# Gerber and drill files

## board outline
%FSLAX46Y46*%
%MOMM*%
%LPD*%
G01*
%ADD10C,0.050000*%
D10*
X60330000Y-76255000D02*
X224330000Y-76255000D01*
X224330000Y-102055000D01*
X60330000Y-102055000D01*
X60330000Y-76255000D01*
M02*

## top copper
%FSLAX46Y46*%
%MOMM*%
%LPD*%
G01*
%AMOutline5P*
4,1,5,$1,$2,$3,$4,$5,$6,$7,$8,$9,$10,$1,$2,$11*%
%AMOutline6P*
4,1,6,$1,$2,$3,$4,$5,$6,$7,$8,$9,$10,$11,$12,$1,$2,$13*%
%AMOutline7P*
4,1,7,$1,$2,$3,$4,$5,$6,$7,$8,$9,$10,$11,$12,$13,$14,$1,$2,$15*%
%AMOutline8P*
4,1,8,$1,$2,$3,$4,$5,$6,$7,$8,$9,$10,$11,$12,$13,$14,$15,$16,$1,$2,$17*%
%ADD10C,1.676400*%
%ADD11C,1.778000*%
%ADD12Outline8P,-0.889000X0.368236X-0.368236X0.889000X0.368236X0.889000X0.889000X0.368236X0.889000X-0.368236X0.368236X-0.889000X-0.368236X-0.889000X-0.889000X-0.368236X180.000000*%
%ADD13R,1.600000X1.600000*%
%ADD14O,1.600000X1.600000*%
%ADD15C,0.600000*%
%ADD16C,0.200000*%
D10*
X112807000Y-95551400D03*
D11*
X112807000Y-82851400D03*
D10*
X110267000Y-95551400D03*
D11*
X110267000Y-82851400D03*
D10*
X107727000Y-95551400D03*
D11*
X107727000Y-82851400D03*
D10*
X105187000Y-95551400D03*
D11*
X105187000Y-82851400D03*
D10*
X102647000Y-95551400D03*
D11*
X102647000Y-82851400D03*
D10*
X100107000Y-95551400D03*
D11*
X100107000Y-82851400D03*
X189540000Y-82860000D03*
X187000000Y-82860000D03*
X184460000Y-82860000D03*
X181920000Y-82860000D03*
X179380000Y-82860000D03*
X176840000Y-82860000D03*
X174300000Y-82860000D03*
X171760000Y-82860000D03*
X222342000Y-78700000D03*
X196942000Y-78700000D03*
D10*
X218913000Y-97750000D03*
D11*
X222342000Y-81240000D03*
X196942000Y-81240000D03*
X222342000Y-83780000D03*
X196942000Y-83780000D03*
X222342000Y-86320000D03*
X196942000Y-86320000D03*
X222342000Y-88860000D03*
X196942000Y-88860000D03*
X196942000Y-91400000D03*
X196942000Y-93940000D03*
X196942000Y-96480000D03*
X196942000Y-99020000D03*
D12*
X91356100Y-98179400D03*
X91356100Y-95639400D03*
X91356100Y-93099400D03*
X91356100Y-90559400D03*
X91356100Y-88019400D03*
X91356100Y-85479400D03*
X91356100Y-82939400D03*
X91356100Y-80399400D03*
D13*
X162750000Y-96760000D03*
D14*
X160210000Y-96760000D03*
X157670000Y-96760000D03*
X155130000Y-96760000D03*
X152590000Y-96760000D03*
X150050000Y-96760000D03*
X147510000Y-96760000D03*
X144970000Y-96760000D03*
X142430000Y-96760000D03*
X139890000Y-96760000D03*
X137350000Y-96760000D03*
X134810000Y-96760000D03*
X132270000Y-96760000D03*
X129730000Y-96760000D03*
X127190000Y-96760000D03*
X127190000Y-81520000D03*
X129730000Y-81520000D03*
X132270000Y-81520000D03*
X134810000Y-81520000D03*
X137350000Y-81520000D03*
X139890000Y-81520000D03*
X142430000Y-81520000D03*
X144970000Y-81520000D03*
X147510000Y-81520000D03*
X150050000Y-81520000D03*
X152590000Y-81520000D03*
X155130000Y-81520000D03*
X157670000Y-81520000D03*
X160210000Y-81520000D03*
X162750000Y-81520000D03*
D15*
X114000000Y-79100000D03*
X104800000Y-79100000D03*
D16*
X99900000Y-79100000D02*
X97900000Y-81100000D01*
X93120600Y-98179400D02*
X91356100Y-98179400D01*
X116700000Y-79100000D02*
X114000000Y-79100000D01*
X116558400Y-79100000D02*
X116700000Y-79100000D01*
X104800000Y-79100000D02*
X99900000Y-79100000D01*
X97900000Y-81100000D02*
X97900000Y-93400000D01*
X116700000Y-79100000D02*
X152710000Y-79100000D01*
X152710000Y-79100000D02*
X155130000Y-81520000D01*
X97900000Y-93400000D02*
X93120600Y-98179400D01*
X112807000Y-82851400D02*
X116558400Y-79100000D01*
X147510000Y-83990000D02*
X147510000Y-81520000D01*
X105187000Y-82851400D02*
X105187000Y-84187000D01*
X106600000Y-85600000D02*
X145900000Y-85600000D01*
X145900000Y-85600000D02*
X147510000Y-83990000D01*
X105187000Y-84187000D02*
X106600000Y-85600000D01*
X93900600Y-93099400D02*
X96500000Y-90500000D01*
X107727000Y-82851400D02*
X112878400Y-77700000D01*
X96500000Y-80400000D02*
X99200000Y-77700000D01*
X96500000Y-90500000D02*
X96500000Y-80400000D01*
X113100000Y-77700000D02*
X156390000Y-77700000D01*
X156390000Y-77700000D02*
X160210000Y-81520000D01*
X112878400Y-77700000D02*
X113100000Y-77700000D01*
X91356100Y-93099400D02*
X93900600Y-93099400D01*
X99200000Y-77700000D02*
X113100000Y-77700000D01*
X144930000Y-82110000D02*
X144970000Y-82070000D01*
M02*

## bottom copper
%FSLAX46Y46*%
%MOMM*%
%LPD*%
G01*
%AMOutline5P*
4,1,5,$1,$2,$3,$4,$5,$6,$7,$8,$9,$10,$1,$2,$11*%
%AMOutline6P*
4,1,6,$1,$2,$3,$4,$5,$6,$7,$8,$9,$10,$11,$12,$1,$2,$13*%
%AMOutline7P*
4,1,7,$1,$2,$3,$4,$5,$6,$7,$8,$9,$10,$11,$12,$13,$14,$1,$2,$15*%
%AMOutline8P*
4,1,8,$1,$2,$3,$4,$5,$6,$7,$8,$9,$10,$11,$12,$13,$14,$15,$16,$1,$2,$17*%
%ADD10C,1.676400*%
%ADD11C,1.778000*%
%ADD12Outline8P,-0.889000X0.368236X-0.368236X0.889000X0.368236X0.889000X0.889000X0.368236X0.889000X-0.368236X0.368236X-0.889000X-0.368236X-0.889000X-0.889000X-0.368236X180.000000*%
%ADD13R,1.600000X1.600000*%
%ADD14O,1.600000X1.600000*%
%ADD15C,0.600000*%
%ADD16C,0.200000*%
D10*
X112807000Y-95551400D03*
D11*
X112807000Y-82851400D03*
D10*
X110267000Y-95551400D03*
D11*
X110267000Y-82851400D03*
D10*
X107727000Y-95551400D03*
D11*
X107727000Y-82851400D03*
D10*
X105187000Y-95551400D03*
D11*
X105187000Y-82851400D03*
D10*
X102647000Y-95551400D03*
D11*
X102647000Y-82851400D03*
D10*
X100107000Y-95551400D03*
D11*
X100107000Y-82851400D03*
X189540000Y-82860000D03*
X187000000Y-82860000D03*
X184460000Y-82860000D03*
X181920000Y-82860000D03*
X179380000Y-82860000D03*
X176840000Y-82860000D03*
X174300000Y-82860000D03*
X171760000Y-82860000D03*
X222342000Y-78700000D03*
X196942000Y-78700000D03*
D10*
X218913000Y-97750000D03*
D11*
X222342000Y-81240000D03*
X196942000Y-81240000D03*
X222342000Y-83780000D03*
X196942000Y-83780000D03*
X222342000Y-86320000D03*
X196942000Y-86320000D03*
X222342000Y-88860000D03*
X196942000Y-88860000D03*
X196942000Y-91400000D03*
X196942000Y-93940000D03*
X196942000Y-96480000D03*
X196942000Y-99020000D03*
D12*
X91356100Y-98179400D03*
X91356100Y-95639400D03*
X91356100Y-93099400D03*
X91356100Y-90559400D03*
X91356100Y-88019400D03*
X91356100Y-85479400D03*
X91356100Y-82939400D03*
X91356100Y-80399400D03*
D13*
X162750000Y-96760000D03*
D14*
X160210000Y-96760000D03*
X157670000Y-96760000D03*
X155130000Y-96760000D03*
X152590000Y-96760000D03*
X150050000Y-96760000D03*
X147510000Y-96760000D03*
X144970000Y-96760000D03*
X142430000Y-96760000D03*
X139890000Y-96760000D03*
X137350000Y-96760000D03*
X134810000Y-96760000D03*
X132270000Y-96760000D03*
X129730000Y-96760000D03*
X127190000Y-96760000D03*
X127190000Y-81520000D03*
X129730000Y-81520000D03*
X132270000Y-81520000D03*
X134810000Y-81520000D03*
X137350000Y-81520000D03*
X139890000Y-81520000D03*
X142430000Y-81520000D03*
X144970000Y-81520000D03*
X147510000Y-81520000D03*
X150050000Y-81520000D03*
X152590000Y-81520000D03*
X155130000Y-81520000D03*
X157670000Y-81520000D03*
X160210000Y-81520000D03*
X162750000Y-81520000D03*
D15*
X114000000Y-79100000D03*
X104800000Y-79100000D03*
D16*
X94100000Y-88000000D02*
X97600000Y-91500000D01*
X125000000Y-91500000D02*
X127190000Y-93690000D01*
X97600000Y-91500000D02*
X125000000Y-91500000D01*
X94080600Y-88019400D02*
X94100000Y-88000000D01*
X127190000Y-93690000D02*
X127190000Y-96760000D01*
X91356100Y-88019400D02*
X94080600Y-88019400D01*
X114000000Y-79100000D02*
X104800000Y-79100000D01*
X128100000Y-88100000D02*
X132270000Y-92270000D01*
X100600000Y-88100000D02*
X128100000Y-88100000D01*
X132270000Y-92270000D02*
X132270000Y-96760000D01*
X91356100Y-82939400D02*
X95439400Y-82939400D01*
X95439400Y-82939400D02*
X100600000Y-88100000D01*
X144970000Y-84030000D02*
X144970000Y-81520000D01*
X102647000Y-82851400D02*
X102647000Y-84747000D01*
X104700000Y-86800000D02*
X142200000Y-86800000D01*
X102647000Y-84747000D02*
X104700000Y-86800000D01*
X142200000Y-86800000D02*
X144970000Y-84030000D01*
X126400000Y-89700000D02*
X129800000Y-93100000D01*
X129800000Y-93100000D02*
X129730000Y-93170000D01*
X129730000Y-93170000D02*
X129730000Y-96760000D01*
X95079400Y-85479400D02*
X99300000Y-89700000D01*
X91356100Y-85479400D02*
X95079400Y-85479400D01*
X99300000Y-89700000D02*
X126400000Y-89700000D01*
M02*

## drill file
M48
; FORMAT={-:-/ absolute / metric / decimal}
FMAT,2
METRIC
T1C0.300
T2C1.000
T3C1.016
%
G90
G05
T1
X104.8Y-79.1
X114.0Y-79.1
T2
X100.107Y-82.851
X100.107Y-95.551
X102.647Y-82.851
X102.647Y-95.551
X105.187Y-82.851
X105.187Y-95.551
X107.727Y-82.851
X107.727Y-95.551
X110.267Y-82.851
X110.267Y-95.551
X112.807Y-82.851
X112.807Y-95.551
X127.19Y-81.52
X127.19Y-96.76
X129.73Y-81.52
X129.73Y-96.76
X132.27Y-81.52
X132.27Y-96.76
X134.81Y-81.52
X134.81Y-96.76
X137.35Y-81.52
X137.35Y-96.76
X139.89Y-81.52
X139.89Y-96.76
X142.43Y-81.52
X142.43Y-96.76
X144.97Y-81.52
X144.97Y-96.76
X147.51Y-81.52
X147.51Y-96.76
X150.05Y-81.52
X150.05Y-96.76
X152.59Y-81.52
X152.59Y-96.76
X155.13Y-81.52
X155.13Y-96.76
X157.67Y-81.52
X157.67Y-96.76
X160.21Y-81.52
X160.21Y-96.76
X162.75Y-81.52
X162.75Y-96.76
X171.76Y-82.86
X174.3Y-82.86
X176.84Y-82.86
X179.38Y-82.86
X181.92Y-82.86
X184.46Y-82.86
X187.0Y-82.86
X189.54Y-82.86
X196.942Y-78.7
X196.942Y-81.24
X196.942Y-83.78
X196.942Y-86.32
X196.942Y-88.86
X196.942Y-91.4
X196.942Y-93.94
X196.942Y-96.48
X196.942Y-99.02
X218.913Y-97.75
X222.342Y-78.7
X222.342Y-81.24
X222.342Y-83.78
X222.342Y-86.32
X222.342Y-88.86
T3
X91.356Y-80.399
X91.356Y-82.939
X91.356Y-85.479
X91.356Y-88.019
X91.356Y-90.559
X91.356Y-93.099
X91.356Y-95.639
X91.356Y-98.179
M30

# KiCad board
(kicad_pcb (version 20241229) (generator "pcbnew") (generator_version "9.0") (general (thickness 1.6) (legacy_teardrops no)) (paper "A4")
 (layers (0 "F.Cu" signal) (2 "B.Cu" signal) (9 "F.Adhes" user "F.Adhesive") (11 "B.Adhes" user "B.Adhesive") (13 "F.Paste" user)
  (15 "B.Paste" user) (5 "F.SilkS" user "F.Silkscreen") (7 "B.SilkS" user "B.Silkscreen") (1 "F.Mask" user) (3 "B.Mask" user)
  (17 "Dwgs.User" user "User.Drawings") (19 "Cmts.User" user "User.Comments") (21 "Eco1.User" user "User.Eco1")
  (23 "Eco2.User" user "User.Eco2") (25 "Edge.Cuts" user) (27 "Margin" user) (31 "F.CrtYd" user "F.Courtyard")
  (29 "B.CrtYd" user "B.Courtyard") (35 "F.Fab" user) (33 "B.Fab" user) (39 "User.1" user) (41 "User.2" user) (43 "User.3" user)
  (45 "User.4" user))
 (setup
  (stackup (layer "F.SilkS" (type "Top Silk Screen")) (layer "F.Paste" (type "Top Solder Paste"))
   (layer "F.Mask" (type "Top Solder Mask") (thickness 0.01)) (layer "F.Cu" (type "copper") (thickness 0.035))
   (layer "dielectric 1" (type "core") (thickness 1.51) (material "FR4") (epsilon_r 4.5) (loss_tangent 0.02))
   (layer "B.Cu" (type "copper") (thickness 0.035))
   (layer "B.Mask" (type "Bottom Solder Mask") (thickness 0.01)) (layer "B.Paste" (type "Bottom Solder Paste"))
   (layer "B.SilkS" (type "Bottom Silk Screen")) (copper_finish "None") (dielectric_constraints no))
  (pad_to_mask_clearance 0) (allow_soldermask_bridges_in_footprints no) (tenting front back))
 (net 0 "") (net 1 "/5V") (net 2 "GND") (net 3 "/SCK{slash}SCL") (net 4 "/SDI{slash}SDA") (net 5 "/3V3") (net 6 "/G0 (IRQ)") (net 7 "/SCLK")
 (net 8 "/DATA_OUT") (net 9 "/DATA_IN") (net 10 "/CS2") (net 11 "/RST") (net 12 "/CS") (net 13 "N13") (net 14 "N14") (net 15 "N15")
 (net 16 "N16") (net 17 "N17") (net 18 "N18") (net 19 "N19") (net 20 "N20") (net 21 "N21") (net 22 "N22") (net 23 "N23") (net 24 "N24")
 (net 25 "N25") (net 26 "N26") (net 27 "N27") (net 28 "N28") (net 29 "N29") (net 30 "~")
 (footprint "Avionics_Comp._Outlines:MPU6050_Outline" (layer "F.Cu") (at 106.63 89.205 180)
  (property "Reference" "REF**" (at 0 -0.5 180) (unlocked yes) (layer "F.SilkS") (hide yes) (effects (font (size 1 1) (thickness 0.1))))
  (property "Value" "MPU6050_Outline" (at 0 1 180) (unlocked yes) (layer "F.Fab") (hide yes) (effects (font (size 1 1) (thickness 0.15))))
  (pad "1" thru_hole circle (at -6.177 -6.3464 270) (size 1.6764 1.6764) (drill 1) (layers "*.Cu" "*.Mask") (remove_unused_layers no)
   (solder_mask_margin 0.0508) (thermal_bridge_angle 0))
  (pad "1" thru_hole circle (at -6.177 6.3536 270) (size 1.778 1.778) (drill 1) (layers "*.Cu" "*.Mask") (remove_unused_layers no)
   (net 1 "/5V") (solder_mask_margin 0.0508) (thermal_bridge_angle 0))
  (pad "2" thru_hole circle (at -3.637 -6.3464 270) (size 1.6764 1.6764) (drill 1) (layers "*.Cu" "*.Mask") (remove_unused_layers no)
   (solder_mask_margin 0.0508) (thermal_bridge_angle 0))
  (pad "2" thru_hole circle (at -3.637 6.3536 270) (size 1.778 1.778) (drill 1) (layers "*.Cu" "*.Mask") (remove_unused_layers no)
   (solder_mask_margin 0.0508) (thermal_bridge_angle 0))
  (pad "3" thru_hole circle (at -1.097 -6.3464 270) (size 1.6764 1.6764) (drill 1) (layers "*.Cu" "*.Mask") (remove_unused_layers no)
   (solder_mask_margin 0.0508) (thermal_bridge_angle 0))
  (pad "3" thru_hole circle (at -1.097 6.3536 270) (size 1.778 1.778) (drill 1) (layers "*.Cu" "*.Mask") (remove_unused_layers no)
   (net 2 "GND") (solder_mask_margin 0.0508) (thermal_bridge_angle 0))
  (pad "4" thru_hole circle (at 1.443 -6.3464 270) (size 1.6764 1.6764) (drill 1) (layers "*.Cu" "*.Mask") (remove_unused_layers no)
   (solder_mask_margin 0.0508) (thermal_bridge_angle 0))
  (pad "4" thru_hole circle (at 1.443 6.3536 270) (size 1.778 1.778) (drill 1) (layers "*.Cu" "*.Mask") (remove_unused_layers no)
   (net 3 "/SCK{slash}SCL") (solder_mask_margin 0.0508) (thermal_bridge_angle 0))
  (pad "5" thru_hole circle (at 3.983 -6.3464 270) (size 1.6764 1.6764) (drill 1) (layers "*.Cu" "*.Mask") (remove_unused_layers no)
   (solder_mask_margin 0.0508) (thermal_bridge_angle 0))
  (pad "5" thru_hole circle (at 3.983 6.3536 270) (size 1.778 1.778) (drill 1) (layers "*.Cu" "*.Mask") (remove_unused_layers no)
   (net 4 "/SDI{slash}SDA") (solder_mask_margin 0.0508) (thermal_bridge_angle 0))
  (pad "6" thru_hole circle (at 6.523 -6.3464 270) (size 1.6764 1.6764) (drill 1) (layers "*.Cu" "*.Mask") (remove_unused_layers no)
   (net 2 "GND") (solder_mask_margin 0.0508) (thermal_bridge_angle 0))
  (pad "6" thru_hole circle (at 6.523 6.3536 270) (size 1.778 1.778) (drill 1) (layers "*.Cu" "*.Mask") (remove_unused_layers no)
   (solder_mask_margin 0.0508) (thermal_bridge_angle 0)))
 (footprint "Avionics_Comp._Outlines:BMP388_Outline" (layer "F.Cu") (at 179.323 85.7136 180)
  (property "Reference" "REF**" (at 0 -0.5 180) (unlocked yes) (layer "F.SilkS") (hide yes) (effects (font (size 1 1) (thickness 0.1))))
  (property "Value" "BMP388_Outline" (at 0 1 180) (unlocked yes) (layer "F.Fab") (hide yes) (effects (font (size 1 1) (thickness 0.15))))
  (pad "1" thru_hole circle (at -10.217 2.8536 270) (size 1.778 1.778) (drill 1) (layers "*.Cu" "*.Mask") (remove_unused_layers no)
   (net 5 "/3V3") (solder_mask_margin 0.0508) (thermal_bridge_angle 0))
  (pad "2" thru_hole circle (at -7.677 2.8536 270) (size 1.778 1.778) (drill 1) (layers "*.Cu" "*.Mask") (remove_unused_layers no)
   (solder_mask_margin 0.0508) (thermal_bridge_angle 0))
  (pad "3" thru_hole circle (at -5.137 2.8536 270) (size 1.778 1.778) (drill 1) (layers "*.Cu" "*.Mask") (remove_unused_layers no)
   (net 2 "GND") (solder_mask_margin 0.0508) (thermal_bridge_angle 0))
  (pad "4" thru_hole circle (at -2.597 2.8536 270) (size 1.778 1.778) (drill 1) (layers "*.Cu" "*.Mask") (remove_unused_layers no)
   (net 3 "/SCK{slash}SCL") (solder_mask_margin 0.0508) (thermal_bridge_angle 0))
  (pad "5" thru_hole circle (at -0.057 2.8536 270) (size 1.778 1.778) (drill 1) (layers "*.Cu" "*.Mask") (remove_unused_layers no)
   (solder_mask_margin 0.0508) (thermal_bridge_angle 0))
  (pad "6" thru_hole circle (at 2.483 2.8536 270) (size 1.778 1.778) (drill 1) (layers "*.Cu" "*.Mask") (remove_unused_layers no)
   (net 4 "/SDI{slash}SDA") (solder_mask_margin 0.0508) (thermal_bridge_angle 0))
  (pad "7" thru_hole circle (at 5.023 2.8536 270) (size 1.778 1.778) (drill 1) (layers "*.Cu" "*.Mask") (remove_unused_layers no)
   (solder_mask_margin 0.0508) (thermal_bridge_angle 0))
  (pad "8" thru_hole circle (at 7.563 2.8536 270) (size 1.778 1.778) (drill 1) (layers "*.Cu" "*.Mask") (remove_unused_layers no)
   (solder_mask_margin 0.0508) (thermal_bridge_angle 0)))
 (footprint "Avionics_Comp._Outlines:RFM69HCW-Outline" (layer "F.Cu") (at 208.65 90.36 -90)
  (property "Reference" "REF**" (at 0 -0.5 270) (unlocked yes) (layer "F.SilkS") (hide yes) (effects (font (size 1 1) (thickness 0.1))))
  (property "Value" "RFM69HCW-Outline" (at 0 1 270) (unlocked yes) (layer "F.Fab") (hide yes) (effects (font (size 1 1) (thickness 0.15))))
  (pad "1" thru_hole circle (at -11.66 -13.692) (size 1.778 1.778) (drill 1) (layers "*.Cu" "*.Mask") (remove_unused_layers no)
   (solder_mask_margin 0.0508) (thermal_bridge_angle 0))
  (pad "1" thru_hole circle (at -11.66 11.708) (size 1.778 1.778) (drill 1) (layers "*.Cu" "*.Mask") (remove_unused_layers no) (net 1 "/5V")
   (solder_mask_margin 0.0508) (thermal_bridge_angle 0))
  (pad "1" thru_hole circle (at 7.39 -10.263) (size 1.6764 1.6764) (drill 1) (layers "*.Cu" "*.Mask") (remove_unused_layers no)
   (solder_mask_margin 0.0508) (thermal_bridge_angle 0))
  (pad "2" thru_hole circle (at -9.12 -13.692) (size 1.778 1.778) (drill 1) (layers "*.Cu" "*.Mask") (remove_unused_layers no)
   (solder_mask_margin 0.0508) (thermal_bridge_angle 0))
  (pad "2" thru_hole circle (at -9.12 11.708) (size 1.778 1.778) (drill 1) (layers "*.Cu" "*.Mask") (remove_unused_layers no) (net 2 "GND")
   (solder_mask_margin 0.0508) (thermal_bridge_angle 0))
  (pad "3" thru_hole circle (at -6.58 -13.692) (size 1.778 1.778) (drill 1) (layers "*.Cu" "*.Mask") (remove_unused_layers no)
   (solder_mask_margin 0.0508) (thermal_bridge_angle 0))
  (pad "3" thru_hole circle (at -6.58 11.708) (size 1.778 1.778) (drill 1) (layers "*.Cu" "*.Mask") (remove_unused_layers no)
   (solder_mask_margin 0.0508) (thermal_bridge_angle 0))
  (pad "4" thru_hole circle (at -4.04 -13.692) (size 1.778 1.778) (drill 1) (layers "*.Cu" "*.Mask") (remove_unused_layers no)
   (solder_mask_margin 0.0508) (thermal_bridge_angle 0))
  (pad "4" thru_hole circle (at -4.04 11.708) (size 1.778 1.778) (drill 1) (layers "*.Cu" "*.Mask") (remove_unused_layers no)
   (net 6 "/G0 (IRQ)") (solder_mask_margin 0.0508) (thermal_bridge_angle 0))
  (pad "5" thru_hole circle (at -1.5 -13.692) (size 1.778 1.778) (drill 1) (layers "*.Cu" "*.Mask") (remove_unused_layers no)
   (solder_mask_margin 0.0508) (thermal_bridge_angle 0))
  (pad "5" thru_hole circle (at -1.5 11.708) (size 1.778 1.778) (drill 1) (layers "*.Cu" "*.Mask") (remove_unused_layers no) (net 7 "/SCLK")
   (solder_mask_margin 0.0508) (thermal_bridge_angle 0))
  (pad "6" thru_hole circle (at 1.04 11.708) (size 1.778 1.778) (drill 1) (layers "*.Cu" "*.Mask") (remove_unused_layers no)
   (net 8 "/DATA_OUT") (solder_mask_margin 0.0508) (thermal_bridge_angle 0))
  (pad "7" thru_hole circle (at 3.58 11.708) (size 1.778 1.778) (drill 1) (layers "*.Cu" "*.Mask") (remove_unused_layers no)
   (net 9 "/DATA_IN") (solder_mask_margin 0.0508) (thermal_bridge_angle 0))
  (pad "8" thru_hole circle (at 6.12 11.708) (size 1.778 1.778) (drill 1) (layers "*.Cu" "*.Mask") (remove_unused_layers no) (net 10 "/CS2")
   (solder_mask_margin 0.0508) (thermal_bridge_angle 0))
  (pad "9" thru_hole circle (at 8.66 11.708) (size 1.778 1.778) (drill 1) (layers "*.Cu" "*.Mask") (remove_unused_layers no) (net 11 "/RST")
   (solder_mask_margin 0.0508) (thermal_bridge_angle 0)))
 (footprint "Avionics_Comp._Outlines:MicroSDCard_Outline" (layer "F.Cu") (at 76.25 88.81)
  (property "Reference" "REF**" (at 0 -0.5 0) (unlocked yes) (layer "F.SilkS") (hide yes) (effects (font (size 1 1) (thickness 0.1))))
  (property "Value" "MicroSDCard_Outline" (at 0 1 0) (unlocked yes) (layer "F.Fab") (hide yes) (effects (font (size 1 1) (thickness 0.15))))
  (pad "1" thru_hole roundrect (at 15.1061 9.3694 180) (size 1.778 1.778) (drill 1.016) (layers "*.Cu" "*.Mask") (remove_unused_layers no)
   (roundrect_rratio 0.25) (chamfer_ratio 0.2928932188) (chamfer top_left top_right bottom_left bottom_right) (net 1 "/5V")
   (solder_mask_margin 0.1016) (thermal_bridge_angle 0))
  (pad "2" thru_hole roundrect (at 15.1061 6.8294 180) (size 1.778 1.778) (drill 1.016) (layers "*.Cu" "*.Mask") (remove_unused_layers no)
   (roundrect_rratio 0.25) (chamfer_ratio 0.2928932188) (chamfer top_left top_right bottom_left bottom_right) (solder_mask_margin 0.1016)
   (thermal_bridge_angle 0))
  (pad "3" thru_hole roundrect (at 15.1061 4.2894 180) (size 1.778 1.778) (drill 1.016) (layers "*.Cu" "*.Mask") (remove_unused_layers no)
   (roundrect_rratio 0.25) (chamfer_ratio 0.2928932188) (chamfer top_left top_right bottom_left bottom_right) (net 2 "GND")
   (solder_mask_margin 0.1016) (thermal_bridge_angle 0))
  (pad "4" thru_hole roundrect (at 15.1061 1.7494 180) (size 1.778 1.778) (drill 1.016) (layers "*.Cu" "*.Mask") (remove_unused_layers no)
   (roundrect_rratio 0.25) (chamfer_ratio 0.2928932188) (chamfer top_left top_right bottom_left bottom_right) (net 7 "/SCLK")
   (solder_mask_margin 0.1016) (thermal_bridge_angle 0))
  (pad "5" thru_hole roundrect (at 15.1061 -0.7906 180) (size 1.778 1.778) (drill 1.016) (layers "*.Cu" "*.Mask") (remove_unused_layers no)
   (roundrect_rratio 0.25) (chamfer_ratio 0.2928932188) (chamfer top_left top_right bottom_left bottom_right) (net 8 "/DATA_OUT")
   (solder_mask_margin 0.1016) (thermal_bridge_angle 0))
  (pad "6" thru_hole roundrect (at 15.1061 -3.3306 180) (size 1.778 1.778) (drill 1.016) (layers "*.Cu" "*.Mask") (remove_unused_layers no)
   (roundrect_rratio 0.25) (chamfer_ratio 0.2928932188) (chamfer top_left top_right bottom_left bottom_right) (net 9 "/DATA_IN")
   (solder_mask_margin 0.1016) (thermal_bridge_angle 0))
  (pad "7" thru_hole roundrect (at 15.1061 -5.8706 180) (size 1.778 1.778) (drill 1.016) (layers "*.Cu" "*.Mask") (remove_unused_layers no)
   (roundrect_rratio 0.25) (chamfer_ratio 0.2928932188) (chamfer top_left top_right bottom_left bottom_right) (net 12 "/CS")
   (solder_mask_margin 0.1016) (thermal_bridge_angle 0))
  (pad "8" thru_hole roundrect (at 15.1061 -8.4106 180) (size 1.778 1.778) (drill 1.016) (layers "*.Cu" "*.Mask") (remove_unused_layers no)
   (roundrect_rratio 0.25) (chamfer_ratio 0.2928932188) (chamfer top_left top_right bottom_left bottom_right) (solder_mask_margin 0.1016)
   (thermal_bridge_angle 0)))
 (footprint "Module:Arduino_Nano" (layer "B.Cu") (at 162.75 96.76 90)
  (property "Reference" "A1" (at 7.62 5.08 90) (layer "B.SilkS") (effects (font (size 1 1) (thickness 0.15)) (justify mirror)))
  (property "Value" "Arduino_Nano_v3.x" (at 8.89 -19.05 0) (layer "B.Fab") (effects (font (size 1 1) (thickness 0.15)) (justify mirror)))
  (pad "1" thru_hole rect (at 0 0 90) (size 1.6 1.6) (drill 1) (layers "*.Cu" "*.Mask") (remove_unused_layers no) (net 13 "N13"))
  (pad "2" thru_hole oval (at 0 -2.54 90) (size 1.6 1.6) (drill 1) (layers "*.Cu" "*.Mask") (remove_unused_layers no) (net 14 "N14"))
  (pad "3" thru_hole oval (at 0 -5.08 90) (size 1.6 1.6) (drill 1) (layers "*.Cu" "*.Mask") (remove_unused_layers no) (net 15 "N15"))
  (pad "4" thru_hole oval (at 0 -7.62 90) (size 1.6 1.6) (drill 1) (layers "*.Cu" "*.Mask") (remove_unused_layers no) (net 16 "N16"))
  (pad "5" thru_hole oval (at 0 -10.16 90) (size 1.6 1.6) (drill 1) (layers "*.Cu" "*.Mask") (remove_unused_layers no) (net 11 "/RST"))
  (pad "6" thru_hole oval (at 0 -12.7 90) (size 1.6 1.6) (drill 1) (layers "*.Cu" "*.Mask") (remove_unused_layers no) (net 6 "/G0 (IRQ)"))
  (pad "7" thru_hole oval (at 0 -15.24 90) (size 1.6 1.6) (drill 1) (layers "*.Cu" "*.Mask") (remove_unused_layers no) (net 10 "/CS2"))
  (pad "8" thru_hole oval (at 0 -17.78 90) (size 1.6 1.6) (drill 1) (layers "*.Cu" "*.Mask") (remove_unused_layers no) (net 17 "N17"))
  (pad "9" thru_hole oval (at 0 -20.32 90) (size 1.6 1.6) (drill 1) (layers "*.Cu" "*.Mask") (remove_unused_layers no) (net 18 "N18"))
  (pad "10" thru_hole oval (at 0 -22.86 90) (size 1.6 1.6) (drill 1) (layers "*.Cu" "*.Mask") (remove_unused_layers no) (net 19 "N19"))
  (pad "11" thru_hole oval (at 0 -25.4 90) (size 1.6 1.6) (drill 1) (layers "*.Cu" "*.Mask") (remove_unused_layers no) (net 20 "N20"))
  (pad "12" thru_hole oval (at 0 -27.94 90) (size 1.6 1.6) (drill 1) (layers "*.Cu" "*.Mask") (remove_unused_layers no) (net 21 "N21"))
  (pad "13" thru_hole oval (at 0 -30.48 90) (size 1.6 1.6) (drill 1) (layers "*.Cu" "*.Mask") (remove_unused_layers no) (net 12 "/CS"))
  (pad "14" thru_hole oval (at 0 -33.02 90) (size 1.6 1.6) (drill 1) (layers "*.Cu" "*.Mask") (remove_unused_layers no) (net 9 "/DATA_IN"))
  (pad "15" thru_hole oval (at 0 -35.56 90) (size 1.6 1.6) (drill 1) (layers "*.Cu" "*.Mask") (remove_unused_layers no) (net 8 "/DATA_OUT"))
  (pad "16" thru_hole oval (at 15.24 -35.56 90) (size 1.6 1.6) (drill 1) (layers "*.Cu" "*.Mask") (remove_unused_layers no) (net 7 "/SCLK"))
  (pad "17" thru_hole oval (at 15.24 -33.02 90) (size 1.6 1.6) (drill 1) (layers "*.Cu" "*.Mask") (remove_unused_layers no) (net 5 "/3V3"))
  (pad "18" thru_hole oval (at 15.24 -30.48 90) (size 1.6 1.6) (drill 1) (layers "*.Cu" "*.Mask") (remove_unused_layers no) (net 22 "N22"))
  (pad "19" thru_hole oval (at 15.24 -27.94 90) (size 1.6 1.6) (drill 1) (layers "*.Cu" "*.Mask") (remove_unused_layers no) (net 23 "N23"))
  (pad "20" thru_hole oval (at 15.24 -25.4 90) (size 1.6 1.6) (drill 1) (layers "*.Cu" "*.Mask") (remove_unused_layers no) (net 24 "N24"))
  (pad "21" thru_hole oval (at 15.24 -22.86 90) (size 1.6 1.6) (drill 1) (layers "*.Cu" "*.Mask") (remove_unused_layers no) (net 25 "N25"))
  (pad "22" thru_hole oval (at 15.24 -20.32 90) (size 1.6 1.6) (drill 1) (layers "*.Cu" "*.Mask") (remove_unused_layers no) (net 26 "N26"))
  (pad "23" thru_hole oval (at 15.24 -17.78 90) (size 1.6 1.6) (drill 1) (layers "*.Cu" "*.Mask") (remove_unused_layers no)
   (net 4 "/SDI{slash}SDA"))
  (pad "24" thru_hole oval (at 15.24 -15.24 90) (size 1.6 1.6) (drill 1) (layers "*.Cu" "*.Mask") (remove_unused_layers no)
   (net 3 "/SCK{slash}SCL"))
  (pad "25" thru_hole oval (at 15.24 -12.7 90) (size 1.6 1.6) (drill 1) (layers "*.Cu" "*.Mask") (remove_unused_layers no) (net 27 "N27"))
  (pad "26" thru_hole oval (at 15.24 -10.16 90) (size 1.6 1.6) (drill 1) (layers "*.Cu" "*.Mask") (remove_unused_layers no) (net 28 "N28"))
  (pad "27" thru_hole oval (at 15.24 -7.62 90) (size 1.6 1.6) (drill 1) (layers "*.Cu" "*.Mask") (remove_unused_layers no) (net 1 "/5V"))
  (pad "28" thru_hole oval (at 15.24 -5.08 90) (size 1.6 1.6) (drill 1) (layers "*.Cu" "*.Mask") (remove_unused_layers no) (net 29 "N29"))
  (pad "29" thru_hole oval (at 15.24 -2.54 90) (size 1.6 1.6) (drill 1) (layers "*.Cu" "*.Mask") (remove_unused_layers no) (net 2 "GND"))
  (pad "30" thru_hole oval (at 15.24 0 90) (size 1.6 1.6) (drill 1) (layers "*.Cu" "*.Mask") (remove_unused_layers no) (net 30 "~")))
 (gr_rect (start 60.33 76.255) (end 224.33 102.055) (stroke (width 0.05) (type default)) (fill no) (layer "Edge.Cuts"))
 (segment (start 94.1 88) (end 97.6 91.5) (width 0.2) (layer "B.Cu") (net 8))
 (segment (start 125 91.5) (end 127.19 93.69) (width 0.2) (layer "B.Cu") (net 8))
 (segment (start 97.6 91.5) (end 125 91.5) (width 0.2) (layer "B.Cu") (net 8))
 (segment (start 94.0806 88.0194) (end 94.1 88) (width 0.2) (layer "B.Cu") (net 8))
 (segment (start 127.19 93.69) (end 127.19 96.76) (width 0.2) (layer "B.Cu") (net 8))
 (segment (start 91.3561 88.0194) (end 94.0806 88.0194) (width 0.2) (layer "B.Cu") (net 8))
 (segment (start 99.9 79.1) (end 97.9 81.1) (width 0.2) (layer "F.Cu") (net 1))
 (segment (start 93.1206 98.1794) (end 91.3561 98.1794) (width 0.2) (layer "F.Cu") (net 1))
 (segment (start 116.7 79.1) (end 114 79.1) (width 0.2) (layer "F.Cu") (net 1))
 (segment (start 116.5584 79.1) (end 116.7 79.1) (width 0.2) (layer "F.Cu") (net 1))
 (segment (start 104.8 79.1) (end 99.9 79.1) (width 0.2) (layer "F.Cu") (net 1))
 (segment (start 97.9 81.1) (end 97.9 93.4) (width 0.2) (layer "F.Cu") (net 1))
 (segment (start 116.7 79.1) (end 152.71 79.1) (width 0.2) (layer "F.Cu") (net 1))
 (segment (start 152.71 79.1) (end 155.13 81.52) (width 0.2) (layer "F.Cu") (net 1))
 (segment (start 97.9 93.4) (end 93.1206 98.1794) (width 0.2) (layer "F.Cu") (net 1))
 (segment (start 112.807 82.8514) (end 116.5584 79.1) (width 0.2) (layer "F.Cu") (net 1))
 (via (at 114 79.1) (size 0.6) (drill 0.3) (layers "F.Cu" "B.Cu") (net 1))
 (via (at 104.8 79.1) (size 0.6) (drill 0.3) (layers "F.Cu" "B.Cu") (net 1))
 (segment (start 114 79.1) (end 104.8 79.1) (width 0.2) (layer "B.Cu") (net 1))
 (segment (start 147.51 83.99) (end 147.51 81.52) (width 0.2) (layer "F.Cu") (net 3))
 (segment (start 105.187 82.8514) (end 105.187 84.187) (width 0.2) (layer "F.Cu") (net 3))
 (segment (start 106.6 85.6) (end 145.9 85.6) (width 0.2) (layer "F.Cu") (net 3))
 (segment (start 145.9 85.6) (end 147.51 83.99) (width 0.2) (layer "F.Cu") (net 3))
 (segment (start 105.187 84.187) (end 106.6 85.6) (width 0.2) (layer "F.Cu") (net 3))
 (segment (start 93.9006 93.0994) (end 96.5 90.5) (width 0.2) (layer "F.Cu") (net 2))
 (segment (start 107.727 82.8514) (end 112.8784 77.7) (width 0.2) (layer "F.Cu") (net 2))
 (segment (start 96.5 80.4) (end 99.2 77.7) (width 0.2) (layer "F.Cu") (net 2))
 (segment (start 96.5 90.5) (end 96.5 80.4) (width 0.2) (layer "F.Cu") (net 2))
 (segment (start 113.1 77.7) (end 156.39 77.7) (width 0.2) (layer "F.Cu") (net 2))
 (segment (start 156.39 77.7) (end 160.21 81.52) (width 0.2) (layer "F.Cu") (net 2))
 (segment (start 112.8784 77.7) (end 113.1 77.7) (width 0.2) (layer "F.Cu") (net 2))
 (segment (start 91.3561 93.0994) (end 93.9006 93.0994) (width 0.2) (layer "F.Cu") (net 2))
 (segment (start 99.2 77.7) (end 113.1 77.7) (width 0.2) (layer "F.Cu") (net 2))
 (segment (start 128.1 88.1) (end 132.27 92.27) (width 0.2) (layer "B.Cu") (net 12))
 (segment (start 100.6 88.1) (end 128.1 88.1) (width 0.2) (layer "B.Cu") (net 12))
 (segment (start 132.27 92.27) (end 132.27 96.76) (width 0.2) (layer "B.Cu") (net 12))
 (segment (start 91.3561 82.9394) (end 95.4394 82.9394) (width 0.2) (layer "B.Cu") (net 12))
 (segment (start 95.4394 82.9394) (end 100.6 88.1) (width 0.2) (layer "B.Cu") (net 12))
 (segment (start 144.93 82.11) (end 144.97 82.07) (width 0.2) (layer "F.Cu") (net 4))
 (segment (start 144.97 84.03) (end 144.97 81.52) (width 0.2) (layer "B.Cu") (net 4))
 (segment (start 102.647 82.8514) (end 102.647 84.747) (width 0.2) (layer "B.Cu") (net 4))
 (segment (start 104.7 86.8) (end 142.2 86.8) (width 0.2) (layer "B.Cu") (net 4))
 (segment (start 102.647 84.747) (end 104.7 86.8) (width 0.2) (layer "B.Cu") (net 4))
 (segment (start 142.2 86.8) (end 144.97 84.03) (width 0.2) (layer "B.Cu") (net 4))
 (segment (start 126.4 89.7) (end 129.8 93.1) (width 0.2) (layer "B.Cu") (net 9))
 (segment (start 129.8 93.1) (end 129.73 93.17) (width 0.2) (layer "B.Cu") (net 9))
 (segment (start 129.73 93.17) (end 129.73 96.76) (width 0.2) (layer "B.Cu") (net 9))
 (segment (start 95.0794 85.4794) (end 99.3 89.7) (width 0.2) (layer "B.Cu") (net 9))
 (segment (start 91.3561 85.4794) (end 95.0794 85.4794) (width 0.2) (layer "B.Cu") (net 9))
 (segment (start 99.3 89.7) (end 126.4 89.7) (width 0.2) (layer "B.Cu") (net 9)))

